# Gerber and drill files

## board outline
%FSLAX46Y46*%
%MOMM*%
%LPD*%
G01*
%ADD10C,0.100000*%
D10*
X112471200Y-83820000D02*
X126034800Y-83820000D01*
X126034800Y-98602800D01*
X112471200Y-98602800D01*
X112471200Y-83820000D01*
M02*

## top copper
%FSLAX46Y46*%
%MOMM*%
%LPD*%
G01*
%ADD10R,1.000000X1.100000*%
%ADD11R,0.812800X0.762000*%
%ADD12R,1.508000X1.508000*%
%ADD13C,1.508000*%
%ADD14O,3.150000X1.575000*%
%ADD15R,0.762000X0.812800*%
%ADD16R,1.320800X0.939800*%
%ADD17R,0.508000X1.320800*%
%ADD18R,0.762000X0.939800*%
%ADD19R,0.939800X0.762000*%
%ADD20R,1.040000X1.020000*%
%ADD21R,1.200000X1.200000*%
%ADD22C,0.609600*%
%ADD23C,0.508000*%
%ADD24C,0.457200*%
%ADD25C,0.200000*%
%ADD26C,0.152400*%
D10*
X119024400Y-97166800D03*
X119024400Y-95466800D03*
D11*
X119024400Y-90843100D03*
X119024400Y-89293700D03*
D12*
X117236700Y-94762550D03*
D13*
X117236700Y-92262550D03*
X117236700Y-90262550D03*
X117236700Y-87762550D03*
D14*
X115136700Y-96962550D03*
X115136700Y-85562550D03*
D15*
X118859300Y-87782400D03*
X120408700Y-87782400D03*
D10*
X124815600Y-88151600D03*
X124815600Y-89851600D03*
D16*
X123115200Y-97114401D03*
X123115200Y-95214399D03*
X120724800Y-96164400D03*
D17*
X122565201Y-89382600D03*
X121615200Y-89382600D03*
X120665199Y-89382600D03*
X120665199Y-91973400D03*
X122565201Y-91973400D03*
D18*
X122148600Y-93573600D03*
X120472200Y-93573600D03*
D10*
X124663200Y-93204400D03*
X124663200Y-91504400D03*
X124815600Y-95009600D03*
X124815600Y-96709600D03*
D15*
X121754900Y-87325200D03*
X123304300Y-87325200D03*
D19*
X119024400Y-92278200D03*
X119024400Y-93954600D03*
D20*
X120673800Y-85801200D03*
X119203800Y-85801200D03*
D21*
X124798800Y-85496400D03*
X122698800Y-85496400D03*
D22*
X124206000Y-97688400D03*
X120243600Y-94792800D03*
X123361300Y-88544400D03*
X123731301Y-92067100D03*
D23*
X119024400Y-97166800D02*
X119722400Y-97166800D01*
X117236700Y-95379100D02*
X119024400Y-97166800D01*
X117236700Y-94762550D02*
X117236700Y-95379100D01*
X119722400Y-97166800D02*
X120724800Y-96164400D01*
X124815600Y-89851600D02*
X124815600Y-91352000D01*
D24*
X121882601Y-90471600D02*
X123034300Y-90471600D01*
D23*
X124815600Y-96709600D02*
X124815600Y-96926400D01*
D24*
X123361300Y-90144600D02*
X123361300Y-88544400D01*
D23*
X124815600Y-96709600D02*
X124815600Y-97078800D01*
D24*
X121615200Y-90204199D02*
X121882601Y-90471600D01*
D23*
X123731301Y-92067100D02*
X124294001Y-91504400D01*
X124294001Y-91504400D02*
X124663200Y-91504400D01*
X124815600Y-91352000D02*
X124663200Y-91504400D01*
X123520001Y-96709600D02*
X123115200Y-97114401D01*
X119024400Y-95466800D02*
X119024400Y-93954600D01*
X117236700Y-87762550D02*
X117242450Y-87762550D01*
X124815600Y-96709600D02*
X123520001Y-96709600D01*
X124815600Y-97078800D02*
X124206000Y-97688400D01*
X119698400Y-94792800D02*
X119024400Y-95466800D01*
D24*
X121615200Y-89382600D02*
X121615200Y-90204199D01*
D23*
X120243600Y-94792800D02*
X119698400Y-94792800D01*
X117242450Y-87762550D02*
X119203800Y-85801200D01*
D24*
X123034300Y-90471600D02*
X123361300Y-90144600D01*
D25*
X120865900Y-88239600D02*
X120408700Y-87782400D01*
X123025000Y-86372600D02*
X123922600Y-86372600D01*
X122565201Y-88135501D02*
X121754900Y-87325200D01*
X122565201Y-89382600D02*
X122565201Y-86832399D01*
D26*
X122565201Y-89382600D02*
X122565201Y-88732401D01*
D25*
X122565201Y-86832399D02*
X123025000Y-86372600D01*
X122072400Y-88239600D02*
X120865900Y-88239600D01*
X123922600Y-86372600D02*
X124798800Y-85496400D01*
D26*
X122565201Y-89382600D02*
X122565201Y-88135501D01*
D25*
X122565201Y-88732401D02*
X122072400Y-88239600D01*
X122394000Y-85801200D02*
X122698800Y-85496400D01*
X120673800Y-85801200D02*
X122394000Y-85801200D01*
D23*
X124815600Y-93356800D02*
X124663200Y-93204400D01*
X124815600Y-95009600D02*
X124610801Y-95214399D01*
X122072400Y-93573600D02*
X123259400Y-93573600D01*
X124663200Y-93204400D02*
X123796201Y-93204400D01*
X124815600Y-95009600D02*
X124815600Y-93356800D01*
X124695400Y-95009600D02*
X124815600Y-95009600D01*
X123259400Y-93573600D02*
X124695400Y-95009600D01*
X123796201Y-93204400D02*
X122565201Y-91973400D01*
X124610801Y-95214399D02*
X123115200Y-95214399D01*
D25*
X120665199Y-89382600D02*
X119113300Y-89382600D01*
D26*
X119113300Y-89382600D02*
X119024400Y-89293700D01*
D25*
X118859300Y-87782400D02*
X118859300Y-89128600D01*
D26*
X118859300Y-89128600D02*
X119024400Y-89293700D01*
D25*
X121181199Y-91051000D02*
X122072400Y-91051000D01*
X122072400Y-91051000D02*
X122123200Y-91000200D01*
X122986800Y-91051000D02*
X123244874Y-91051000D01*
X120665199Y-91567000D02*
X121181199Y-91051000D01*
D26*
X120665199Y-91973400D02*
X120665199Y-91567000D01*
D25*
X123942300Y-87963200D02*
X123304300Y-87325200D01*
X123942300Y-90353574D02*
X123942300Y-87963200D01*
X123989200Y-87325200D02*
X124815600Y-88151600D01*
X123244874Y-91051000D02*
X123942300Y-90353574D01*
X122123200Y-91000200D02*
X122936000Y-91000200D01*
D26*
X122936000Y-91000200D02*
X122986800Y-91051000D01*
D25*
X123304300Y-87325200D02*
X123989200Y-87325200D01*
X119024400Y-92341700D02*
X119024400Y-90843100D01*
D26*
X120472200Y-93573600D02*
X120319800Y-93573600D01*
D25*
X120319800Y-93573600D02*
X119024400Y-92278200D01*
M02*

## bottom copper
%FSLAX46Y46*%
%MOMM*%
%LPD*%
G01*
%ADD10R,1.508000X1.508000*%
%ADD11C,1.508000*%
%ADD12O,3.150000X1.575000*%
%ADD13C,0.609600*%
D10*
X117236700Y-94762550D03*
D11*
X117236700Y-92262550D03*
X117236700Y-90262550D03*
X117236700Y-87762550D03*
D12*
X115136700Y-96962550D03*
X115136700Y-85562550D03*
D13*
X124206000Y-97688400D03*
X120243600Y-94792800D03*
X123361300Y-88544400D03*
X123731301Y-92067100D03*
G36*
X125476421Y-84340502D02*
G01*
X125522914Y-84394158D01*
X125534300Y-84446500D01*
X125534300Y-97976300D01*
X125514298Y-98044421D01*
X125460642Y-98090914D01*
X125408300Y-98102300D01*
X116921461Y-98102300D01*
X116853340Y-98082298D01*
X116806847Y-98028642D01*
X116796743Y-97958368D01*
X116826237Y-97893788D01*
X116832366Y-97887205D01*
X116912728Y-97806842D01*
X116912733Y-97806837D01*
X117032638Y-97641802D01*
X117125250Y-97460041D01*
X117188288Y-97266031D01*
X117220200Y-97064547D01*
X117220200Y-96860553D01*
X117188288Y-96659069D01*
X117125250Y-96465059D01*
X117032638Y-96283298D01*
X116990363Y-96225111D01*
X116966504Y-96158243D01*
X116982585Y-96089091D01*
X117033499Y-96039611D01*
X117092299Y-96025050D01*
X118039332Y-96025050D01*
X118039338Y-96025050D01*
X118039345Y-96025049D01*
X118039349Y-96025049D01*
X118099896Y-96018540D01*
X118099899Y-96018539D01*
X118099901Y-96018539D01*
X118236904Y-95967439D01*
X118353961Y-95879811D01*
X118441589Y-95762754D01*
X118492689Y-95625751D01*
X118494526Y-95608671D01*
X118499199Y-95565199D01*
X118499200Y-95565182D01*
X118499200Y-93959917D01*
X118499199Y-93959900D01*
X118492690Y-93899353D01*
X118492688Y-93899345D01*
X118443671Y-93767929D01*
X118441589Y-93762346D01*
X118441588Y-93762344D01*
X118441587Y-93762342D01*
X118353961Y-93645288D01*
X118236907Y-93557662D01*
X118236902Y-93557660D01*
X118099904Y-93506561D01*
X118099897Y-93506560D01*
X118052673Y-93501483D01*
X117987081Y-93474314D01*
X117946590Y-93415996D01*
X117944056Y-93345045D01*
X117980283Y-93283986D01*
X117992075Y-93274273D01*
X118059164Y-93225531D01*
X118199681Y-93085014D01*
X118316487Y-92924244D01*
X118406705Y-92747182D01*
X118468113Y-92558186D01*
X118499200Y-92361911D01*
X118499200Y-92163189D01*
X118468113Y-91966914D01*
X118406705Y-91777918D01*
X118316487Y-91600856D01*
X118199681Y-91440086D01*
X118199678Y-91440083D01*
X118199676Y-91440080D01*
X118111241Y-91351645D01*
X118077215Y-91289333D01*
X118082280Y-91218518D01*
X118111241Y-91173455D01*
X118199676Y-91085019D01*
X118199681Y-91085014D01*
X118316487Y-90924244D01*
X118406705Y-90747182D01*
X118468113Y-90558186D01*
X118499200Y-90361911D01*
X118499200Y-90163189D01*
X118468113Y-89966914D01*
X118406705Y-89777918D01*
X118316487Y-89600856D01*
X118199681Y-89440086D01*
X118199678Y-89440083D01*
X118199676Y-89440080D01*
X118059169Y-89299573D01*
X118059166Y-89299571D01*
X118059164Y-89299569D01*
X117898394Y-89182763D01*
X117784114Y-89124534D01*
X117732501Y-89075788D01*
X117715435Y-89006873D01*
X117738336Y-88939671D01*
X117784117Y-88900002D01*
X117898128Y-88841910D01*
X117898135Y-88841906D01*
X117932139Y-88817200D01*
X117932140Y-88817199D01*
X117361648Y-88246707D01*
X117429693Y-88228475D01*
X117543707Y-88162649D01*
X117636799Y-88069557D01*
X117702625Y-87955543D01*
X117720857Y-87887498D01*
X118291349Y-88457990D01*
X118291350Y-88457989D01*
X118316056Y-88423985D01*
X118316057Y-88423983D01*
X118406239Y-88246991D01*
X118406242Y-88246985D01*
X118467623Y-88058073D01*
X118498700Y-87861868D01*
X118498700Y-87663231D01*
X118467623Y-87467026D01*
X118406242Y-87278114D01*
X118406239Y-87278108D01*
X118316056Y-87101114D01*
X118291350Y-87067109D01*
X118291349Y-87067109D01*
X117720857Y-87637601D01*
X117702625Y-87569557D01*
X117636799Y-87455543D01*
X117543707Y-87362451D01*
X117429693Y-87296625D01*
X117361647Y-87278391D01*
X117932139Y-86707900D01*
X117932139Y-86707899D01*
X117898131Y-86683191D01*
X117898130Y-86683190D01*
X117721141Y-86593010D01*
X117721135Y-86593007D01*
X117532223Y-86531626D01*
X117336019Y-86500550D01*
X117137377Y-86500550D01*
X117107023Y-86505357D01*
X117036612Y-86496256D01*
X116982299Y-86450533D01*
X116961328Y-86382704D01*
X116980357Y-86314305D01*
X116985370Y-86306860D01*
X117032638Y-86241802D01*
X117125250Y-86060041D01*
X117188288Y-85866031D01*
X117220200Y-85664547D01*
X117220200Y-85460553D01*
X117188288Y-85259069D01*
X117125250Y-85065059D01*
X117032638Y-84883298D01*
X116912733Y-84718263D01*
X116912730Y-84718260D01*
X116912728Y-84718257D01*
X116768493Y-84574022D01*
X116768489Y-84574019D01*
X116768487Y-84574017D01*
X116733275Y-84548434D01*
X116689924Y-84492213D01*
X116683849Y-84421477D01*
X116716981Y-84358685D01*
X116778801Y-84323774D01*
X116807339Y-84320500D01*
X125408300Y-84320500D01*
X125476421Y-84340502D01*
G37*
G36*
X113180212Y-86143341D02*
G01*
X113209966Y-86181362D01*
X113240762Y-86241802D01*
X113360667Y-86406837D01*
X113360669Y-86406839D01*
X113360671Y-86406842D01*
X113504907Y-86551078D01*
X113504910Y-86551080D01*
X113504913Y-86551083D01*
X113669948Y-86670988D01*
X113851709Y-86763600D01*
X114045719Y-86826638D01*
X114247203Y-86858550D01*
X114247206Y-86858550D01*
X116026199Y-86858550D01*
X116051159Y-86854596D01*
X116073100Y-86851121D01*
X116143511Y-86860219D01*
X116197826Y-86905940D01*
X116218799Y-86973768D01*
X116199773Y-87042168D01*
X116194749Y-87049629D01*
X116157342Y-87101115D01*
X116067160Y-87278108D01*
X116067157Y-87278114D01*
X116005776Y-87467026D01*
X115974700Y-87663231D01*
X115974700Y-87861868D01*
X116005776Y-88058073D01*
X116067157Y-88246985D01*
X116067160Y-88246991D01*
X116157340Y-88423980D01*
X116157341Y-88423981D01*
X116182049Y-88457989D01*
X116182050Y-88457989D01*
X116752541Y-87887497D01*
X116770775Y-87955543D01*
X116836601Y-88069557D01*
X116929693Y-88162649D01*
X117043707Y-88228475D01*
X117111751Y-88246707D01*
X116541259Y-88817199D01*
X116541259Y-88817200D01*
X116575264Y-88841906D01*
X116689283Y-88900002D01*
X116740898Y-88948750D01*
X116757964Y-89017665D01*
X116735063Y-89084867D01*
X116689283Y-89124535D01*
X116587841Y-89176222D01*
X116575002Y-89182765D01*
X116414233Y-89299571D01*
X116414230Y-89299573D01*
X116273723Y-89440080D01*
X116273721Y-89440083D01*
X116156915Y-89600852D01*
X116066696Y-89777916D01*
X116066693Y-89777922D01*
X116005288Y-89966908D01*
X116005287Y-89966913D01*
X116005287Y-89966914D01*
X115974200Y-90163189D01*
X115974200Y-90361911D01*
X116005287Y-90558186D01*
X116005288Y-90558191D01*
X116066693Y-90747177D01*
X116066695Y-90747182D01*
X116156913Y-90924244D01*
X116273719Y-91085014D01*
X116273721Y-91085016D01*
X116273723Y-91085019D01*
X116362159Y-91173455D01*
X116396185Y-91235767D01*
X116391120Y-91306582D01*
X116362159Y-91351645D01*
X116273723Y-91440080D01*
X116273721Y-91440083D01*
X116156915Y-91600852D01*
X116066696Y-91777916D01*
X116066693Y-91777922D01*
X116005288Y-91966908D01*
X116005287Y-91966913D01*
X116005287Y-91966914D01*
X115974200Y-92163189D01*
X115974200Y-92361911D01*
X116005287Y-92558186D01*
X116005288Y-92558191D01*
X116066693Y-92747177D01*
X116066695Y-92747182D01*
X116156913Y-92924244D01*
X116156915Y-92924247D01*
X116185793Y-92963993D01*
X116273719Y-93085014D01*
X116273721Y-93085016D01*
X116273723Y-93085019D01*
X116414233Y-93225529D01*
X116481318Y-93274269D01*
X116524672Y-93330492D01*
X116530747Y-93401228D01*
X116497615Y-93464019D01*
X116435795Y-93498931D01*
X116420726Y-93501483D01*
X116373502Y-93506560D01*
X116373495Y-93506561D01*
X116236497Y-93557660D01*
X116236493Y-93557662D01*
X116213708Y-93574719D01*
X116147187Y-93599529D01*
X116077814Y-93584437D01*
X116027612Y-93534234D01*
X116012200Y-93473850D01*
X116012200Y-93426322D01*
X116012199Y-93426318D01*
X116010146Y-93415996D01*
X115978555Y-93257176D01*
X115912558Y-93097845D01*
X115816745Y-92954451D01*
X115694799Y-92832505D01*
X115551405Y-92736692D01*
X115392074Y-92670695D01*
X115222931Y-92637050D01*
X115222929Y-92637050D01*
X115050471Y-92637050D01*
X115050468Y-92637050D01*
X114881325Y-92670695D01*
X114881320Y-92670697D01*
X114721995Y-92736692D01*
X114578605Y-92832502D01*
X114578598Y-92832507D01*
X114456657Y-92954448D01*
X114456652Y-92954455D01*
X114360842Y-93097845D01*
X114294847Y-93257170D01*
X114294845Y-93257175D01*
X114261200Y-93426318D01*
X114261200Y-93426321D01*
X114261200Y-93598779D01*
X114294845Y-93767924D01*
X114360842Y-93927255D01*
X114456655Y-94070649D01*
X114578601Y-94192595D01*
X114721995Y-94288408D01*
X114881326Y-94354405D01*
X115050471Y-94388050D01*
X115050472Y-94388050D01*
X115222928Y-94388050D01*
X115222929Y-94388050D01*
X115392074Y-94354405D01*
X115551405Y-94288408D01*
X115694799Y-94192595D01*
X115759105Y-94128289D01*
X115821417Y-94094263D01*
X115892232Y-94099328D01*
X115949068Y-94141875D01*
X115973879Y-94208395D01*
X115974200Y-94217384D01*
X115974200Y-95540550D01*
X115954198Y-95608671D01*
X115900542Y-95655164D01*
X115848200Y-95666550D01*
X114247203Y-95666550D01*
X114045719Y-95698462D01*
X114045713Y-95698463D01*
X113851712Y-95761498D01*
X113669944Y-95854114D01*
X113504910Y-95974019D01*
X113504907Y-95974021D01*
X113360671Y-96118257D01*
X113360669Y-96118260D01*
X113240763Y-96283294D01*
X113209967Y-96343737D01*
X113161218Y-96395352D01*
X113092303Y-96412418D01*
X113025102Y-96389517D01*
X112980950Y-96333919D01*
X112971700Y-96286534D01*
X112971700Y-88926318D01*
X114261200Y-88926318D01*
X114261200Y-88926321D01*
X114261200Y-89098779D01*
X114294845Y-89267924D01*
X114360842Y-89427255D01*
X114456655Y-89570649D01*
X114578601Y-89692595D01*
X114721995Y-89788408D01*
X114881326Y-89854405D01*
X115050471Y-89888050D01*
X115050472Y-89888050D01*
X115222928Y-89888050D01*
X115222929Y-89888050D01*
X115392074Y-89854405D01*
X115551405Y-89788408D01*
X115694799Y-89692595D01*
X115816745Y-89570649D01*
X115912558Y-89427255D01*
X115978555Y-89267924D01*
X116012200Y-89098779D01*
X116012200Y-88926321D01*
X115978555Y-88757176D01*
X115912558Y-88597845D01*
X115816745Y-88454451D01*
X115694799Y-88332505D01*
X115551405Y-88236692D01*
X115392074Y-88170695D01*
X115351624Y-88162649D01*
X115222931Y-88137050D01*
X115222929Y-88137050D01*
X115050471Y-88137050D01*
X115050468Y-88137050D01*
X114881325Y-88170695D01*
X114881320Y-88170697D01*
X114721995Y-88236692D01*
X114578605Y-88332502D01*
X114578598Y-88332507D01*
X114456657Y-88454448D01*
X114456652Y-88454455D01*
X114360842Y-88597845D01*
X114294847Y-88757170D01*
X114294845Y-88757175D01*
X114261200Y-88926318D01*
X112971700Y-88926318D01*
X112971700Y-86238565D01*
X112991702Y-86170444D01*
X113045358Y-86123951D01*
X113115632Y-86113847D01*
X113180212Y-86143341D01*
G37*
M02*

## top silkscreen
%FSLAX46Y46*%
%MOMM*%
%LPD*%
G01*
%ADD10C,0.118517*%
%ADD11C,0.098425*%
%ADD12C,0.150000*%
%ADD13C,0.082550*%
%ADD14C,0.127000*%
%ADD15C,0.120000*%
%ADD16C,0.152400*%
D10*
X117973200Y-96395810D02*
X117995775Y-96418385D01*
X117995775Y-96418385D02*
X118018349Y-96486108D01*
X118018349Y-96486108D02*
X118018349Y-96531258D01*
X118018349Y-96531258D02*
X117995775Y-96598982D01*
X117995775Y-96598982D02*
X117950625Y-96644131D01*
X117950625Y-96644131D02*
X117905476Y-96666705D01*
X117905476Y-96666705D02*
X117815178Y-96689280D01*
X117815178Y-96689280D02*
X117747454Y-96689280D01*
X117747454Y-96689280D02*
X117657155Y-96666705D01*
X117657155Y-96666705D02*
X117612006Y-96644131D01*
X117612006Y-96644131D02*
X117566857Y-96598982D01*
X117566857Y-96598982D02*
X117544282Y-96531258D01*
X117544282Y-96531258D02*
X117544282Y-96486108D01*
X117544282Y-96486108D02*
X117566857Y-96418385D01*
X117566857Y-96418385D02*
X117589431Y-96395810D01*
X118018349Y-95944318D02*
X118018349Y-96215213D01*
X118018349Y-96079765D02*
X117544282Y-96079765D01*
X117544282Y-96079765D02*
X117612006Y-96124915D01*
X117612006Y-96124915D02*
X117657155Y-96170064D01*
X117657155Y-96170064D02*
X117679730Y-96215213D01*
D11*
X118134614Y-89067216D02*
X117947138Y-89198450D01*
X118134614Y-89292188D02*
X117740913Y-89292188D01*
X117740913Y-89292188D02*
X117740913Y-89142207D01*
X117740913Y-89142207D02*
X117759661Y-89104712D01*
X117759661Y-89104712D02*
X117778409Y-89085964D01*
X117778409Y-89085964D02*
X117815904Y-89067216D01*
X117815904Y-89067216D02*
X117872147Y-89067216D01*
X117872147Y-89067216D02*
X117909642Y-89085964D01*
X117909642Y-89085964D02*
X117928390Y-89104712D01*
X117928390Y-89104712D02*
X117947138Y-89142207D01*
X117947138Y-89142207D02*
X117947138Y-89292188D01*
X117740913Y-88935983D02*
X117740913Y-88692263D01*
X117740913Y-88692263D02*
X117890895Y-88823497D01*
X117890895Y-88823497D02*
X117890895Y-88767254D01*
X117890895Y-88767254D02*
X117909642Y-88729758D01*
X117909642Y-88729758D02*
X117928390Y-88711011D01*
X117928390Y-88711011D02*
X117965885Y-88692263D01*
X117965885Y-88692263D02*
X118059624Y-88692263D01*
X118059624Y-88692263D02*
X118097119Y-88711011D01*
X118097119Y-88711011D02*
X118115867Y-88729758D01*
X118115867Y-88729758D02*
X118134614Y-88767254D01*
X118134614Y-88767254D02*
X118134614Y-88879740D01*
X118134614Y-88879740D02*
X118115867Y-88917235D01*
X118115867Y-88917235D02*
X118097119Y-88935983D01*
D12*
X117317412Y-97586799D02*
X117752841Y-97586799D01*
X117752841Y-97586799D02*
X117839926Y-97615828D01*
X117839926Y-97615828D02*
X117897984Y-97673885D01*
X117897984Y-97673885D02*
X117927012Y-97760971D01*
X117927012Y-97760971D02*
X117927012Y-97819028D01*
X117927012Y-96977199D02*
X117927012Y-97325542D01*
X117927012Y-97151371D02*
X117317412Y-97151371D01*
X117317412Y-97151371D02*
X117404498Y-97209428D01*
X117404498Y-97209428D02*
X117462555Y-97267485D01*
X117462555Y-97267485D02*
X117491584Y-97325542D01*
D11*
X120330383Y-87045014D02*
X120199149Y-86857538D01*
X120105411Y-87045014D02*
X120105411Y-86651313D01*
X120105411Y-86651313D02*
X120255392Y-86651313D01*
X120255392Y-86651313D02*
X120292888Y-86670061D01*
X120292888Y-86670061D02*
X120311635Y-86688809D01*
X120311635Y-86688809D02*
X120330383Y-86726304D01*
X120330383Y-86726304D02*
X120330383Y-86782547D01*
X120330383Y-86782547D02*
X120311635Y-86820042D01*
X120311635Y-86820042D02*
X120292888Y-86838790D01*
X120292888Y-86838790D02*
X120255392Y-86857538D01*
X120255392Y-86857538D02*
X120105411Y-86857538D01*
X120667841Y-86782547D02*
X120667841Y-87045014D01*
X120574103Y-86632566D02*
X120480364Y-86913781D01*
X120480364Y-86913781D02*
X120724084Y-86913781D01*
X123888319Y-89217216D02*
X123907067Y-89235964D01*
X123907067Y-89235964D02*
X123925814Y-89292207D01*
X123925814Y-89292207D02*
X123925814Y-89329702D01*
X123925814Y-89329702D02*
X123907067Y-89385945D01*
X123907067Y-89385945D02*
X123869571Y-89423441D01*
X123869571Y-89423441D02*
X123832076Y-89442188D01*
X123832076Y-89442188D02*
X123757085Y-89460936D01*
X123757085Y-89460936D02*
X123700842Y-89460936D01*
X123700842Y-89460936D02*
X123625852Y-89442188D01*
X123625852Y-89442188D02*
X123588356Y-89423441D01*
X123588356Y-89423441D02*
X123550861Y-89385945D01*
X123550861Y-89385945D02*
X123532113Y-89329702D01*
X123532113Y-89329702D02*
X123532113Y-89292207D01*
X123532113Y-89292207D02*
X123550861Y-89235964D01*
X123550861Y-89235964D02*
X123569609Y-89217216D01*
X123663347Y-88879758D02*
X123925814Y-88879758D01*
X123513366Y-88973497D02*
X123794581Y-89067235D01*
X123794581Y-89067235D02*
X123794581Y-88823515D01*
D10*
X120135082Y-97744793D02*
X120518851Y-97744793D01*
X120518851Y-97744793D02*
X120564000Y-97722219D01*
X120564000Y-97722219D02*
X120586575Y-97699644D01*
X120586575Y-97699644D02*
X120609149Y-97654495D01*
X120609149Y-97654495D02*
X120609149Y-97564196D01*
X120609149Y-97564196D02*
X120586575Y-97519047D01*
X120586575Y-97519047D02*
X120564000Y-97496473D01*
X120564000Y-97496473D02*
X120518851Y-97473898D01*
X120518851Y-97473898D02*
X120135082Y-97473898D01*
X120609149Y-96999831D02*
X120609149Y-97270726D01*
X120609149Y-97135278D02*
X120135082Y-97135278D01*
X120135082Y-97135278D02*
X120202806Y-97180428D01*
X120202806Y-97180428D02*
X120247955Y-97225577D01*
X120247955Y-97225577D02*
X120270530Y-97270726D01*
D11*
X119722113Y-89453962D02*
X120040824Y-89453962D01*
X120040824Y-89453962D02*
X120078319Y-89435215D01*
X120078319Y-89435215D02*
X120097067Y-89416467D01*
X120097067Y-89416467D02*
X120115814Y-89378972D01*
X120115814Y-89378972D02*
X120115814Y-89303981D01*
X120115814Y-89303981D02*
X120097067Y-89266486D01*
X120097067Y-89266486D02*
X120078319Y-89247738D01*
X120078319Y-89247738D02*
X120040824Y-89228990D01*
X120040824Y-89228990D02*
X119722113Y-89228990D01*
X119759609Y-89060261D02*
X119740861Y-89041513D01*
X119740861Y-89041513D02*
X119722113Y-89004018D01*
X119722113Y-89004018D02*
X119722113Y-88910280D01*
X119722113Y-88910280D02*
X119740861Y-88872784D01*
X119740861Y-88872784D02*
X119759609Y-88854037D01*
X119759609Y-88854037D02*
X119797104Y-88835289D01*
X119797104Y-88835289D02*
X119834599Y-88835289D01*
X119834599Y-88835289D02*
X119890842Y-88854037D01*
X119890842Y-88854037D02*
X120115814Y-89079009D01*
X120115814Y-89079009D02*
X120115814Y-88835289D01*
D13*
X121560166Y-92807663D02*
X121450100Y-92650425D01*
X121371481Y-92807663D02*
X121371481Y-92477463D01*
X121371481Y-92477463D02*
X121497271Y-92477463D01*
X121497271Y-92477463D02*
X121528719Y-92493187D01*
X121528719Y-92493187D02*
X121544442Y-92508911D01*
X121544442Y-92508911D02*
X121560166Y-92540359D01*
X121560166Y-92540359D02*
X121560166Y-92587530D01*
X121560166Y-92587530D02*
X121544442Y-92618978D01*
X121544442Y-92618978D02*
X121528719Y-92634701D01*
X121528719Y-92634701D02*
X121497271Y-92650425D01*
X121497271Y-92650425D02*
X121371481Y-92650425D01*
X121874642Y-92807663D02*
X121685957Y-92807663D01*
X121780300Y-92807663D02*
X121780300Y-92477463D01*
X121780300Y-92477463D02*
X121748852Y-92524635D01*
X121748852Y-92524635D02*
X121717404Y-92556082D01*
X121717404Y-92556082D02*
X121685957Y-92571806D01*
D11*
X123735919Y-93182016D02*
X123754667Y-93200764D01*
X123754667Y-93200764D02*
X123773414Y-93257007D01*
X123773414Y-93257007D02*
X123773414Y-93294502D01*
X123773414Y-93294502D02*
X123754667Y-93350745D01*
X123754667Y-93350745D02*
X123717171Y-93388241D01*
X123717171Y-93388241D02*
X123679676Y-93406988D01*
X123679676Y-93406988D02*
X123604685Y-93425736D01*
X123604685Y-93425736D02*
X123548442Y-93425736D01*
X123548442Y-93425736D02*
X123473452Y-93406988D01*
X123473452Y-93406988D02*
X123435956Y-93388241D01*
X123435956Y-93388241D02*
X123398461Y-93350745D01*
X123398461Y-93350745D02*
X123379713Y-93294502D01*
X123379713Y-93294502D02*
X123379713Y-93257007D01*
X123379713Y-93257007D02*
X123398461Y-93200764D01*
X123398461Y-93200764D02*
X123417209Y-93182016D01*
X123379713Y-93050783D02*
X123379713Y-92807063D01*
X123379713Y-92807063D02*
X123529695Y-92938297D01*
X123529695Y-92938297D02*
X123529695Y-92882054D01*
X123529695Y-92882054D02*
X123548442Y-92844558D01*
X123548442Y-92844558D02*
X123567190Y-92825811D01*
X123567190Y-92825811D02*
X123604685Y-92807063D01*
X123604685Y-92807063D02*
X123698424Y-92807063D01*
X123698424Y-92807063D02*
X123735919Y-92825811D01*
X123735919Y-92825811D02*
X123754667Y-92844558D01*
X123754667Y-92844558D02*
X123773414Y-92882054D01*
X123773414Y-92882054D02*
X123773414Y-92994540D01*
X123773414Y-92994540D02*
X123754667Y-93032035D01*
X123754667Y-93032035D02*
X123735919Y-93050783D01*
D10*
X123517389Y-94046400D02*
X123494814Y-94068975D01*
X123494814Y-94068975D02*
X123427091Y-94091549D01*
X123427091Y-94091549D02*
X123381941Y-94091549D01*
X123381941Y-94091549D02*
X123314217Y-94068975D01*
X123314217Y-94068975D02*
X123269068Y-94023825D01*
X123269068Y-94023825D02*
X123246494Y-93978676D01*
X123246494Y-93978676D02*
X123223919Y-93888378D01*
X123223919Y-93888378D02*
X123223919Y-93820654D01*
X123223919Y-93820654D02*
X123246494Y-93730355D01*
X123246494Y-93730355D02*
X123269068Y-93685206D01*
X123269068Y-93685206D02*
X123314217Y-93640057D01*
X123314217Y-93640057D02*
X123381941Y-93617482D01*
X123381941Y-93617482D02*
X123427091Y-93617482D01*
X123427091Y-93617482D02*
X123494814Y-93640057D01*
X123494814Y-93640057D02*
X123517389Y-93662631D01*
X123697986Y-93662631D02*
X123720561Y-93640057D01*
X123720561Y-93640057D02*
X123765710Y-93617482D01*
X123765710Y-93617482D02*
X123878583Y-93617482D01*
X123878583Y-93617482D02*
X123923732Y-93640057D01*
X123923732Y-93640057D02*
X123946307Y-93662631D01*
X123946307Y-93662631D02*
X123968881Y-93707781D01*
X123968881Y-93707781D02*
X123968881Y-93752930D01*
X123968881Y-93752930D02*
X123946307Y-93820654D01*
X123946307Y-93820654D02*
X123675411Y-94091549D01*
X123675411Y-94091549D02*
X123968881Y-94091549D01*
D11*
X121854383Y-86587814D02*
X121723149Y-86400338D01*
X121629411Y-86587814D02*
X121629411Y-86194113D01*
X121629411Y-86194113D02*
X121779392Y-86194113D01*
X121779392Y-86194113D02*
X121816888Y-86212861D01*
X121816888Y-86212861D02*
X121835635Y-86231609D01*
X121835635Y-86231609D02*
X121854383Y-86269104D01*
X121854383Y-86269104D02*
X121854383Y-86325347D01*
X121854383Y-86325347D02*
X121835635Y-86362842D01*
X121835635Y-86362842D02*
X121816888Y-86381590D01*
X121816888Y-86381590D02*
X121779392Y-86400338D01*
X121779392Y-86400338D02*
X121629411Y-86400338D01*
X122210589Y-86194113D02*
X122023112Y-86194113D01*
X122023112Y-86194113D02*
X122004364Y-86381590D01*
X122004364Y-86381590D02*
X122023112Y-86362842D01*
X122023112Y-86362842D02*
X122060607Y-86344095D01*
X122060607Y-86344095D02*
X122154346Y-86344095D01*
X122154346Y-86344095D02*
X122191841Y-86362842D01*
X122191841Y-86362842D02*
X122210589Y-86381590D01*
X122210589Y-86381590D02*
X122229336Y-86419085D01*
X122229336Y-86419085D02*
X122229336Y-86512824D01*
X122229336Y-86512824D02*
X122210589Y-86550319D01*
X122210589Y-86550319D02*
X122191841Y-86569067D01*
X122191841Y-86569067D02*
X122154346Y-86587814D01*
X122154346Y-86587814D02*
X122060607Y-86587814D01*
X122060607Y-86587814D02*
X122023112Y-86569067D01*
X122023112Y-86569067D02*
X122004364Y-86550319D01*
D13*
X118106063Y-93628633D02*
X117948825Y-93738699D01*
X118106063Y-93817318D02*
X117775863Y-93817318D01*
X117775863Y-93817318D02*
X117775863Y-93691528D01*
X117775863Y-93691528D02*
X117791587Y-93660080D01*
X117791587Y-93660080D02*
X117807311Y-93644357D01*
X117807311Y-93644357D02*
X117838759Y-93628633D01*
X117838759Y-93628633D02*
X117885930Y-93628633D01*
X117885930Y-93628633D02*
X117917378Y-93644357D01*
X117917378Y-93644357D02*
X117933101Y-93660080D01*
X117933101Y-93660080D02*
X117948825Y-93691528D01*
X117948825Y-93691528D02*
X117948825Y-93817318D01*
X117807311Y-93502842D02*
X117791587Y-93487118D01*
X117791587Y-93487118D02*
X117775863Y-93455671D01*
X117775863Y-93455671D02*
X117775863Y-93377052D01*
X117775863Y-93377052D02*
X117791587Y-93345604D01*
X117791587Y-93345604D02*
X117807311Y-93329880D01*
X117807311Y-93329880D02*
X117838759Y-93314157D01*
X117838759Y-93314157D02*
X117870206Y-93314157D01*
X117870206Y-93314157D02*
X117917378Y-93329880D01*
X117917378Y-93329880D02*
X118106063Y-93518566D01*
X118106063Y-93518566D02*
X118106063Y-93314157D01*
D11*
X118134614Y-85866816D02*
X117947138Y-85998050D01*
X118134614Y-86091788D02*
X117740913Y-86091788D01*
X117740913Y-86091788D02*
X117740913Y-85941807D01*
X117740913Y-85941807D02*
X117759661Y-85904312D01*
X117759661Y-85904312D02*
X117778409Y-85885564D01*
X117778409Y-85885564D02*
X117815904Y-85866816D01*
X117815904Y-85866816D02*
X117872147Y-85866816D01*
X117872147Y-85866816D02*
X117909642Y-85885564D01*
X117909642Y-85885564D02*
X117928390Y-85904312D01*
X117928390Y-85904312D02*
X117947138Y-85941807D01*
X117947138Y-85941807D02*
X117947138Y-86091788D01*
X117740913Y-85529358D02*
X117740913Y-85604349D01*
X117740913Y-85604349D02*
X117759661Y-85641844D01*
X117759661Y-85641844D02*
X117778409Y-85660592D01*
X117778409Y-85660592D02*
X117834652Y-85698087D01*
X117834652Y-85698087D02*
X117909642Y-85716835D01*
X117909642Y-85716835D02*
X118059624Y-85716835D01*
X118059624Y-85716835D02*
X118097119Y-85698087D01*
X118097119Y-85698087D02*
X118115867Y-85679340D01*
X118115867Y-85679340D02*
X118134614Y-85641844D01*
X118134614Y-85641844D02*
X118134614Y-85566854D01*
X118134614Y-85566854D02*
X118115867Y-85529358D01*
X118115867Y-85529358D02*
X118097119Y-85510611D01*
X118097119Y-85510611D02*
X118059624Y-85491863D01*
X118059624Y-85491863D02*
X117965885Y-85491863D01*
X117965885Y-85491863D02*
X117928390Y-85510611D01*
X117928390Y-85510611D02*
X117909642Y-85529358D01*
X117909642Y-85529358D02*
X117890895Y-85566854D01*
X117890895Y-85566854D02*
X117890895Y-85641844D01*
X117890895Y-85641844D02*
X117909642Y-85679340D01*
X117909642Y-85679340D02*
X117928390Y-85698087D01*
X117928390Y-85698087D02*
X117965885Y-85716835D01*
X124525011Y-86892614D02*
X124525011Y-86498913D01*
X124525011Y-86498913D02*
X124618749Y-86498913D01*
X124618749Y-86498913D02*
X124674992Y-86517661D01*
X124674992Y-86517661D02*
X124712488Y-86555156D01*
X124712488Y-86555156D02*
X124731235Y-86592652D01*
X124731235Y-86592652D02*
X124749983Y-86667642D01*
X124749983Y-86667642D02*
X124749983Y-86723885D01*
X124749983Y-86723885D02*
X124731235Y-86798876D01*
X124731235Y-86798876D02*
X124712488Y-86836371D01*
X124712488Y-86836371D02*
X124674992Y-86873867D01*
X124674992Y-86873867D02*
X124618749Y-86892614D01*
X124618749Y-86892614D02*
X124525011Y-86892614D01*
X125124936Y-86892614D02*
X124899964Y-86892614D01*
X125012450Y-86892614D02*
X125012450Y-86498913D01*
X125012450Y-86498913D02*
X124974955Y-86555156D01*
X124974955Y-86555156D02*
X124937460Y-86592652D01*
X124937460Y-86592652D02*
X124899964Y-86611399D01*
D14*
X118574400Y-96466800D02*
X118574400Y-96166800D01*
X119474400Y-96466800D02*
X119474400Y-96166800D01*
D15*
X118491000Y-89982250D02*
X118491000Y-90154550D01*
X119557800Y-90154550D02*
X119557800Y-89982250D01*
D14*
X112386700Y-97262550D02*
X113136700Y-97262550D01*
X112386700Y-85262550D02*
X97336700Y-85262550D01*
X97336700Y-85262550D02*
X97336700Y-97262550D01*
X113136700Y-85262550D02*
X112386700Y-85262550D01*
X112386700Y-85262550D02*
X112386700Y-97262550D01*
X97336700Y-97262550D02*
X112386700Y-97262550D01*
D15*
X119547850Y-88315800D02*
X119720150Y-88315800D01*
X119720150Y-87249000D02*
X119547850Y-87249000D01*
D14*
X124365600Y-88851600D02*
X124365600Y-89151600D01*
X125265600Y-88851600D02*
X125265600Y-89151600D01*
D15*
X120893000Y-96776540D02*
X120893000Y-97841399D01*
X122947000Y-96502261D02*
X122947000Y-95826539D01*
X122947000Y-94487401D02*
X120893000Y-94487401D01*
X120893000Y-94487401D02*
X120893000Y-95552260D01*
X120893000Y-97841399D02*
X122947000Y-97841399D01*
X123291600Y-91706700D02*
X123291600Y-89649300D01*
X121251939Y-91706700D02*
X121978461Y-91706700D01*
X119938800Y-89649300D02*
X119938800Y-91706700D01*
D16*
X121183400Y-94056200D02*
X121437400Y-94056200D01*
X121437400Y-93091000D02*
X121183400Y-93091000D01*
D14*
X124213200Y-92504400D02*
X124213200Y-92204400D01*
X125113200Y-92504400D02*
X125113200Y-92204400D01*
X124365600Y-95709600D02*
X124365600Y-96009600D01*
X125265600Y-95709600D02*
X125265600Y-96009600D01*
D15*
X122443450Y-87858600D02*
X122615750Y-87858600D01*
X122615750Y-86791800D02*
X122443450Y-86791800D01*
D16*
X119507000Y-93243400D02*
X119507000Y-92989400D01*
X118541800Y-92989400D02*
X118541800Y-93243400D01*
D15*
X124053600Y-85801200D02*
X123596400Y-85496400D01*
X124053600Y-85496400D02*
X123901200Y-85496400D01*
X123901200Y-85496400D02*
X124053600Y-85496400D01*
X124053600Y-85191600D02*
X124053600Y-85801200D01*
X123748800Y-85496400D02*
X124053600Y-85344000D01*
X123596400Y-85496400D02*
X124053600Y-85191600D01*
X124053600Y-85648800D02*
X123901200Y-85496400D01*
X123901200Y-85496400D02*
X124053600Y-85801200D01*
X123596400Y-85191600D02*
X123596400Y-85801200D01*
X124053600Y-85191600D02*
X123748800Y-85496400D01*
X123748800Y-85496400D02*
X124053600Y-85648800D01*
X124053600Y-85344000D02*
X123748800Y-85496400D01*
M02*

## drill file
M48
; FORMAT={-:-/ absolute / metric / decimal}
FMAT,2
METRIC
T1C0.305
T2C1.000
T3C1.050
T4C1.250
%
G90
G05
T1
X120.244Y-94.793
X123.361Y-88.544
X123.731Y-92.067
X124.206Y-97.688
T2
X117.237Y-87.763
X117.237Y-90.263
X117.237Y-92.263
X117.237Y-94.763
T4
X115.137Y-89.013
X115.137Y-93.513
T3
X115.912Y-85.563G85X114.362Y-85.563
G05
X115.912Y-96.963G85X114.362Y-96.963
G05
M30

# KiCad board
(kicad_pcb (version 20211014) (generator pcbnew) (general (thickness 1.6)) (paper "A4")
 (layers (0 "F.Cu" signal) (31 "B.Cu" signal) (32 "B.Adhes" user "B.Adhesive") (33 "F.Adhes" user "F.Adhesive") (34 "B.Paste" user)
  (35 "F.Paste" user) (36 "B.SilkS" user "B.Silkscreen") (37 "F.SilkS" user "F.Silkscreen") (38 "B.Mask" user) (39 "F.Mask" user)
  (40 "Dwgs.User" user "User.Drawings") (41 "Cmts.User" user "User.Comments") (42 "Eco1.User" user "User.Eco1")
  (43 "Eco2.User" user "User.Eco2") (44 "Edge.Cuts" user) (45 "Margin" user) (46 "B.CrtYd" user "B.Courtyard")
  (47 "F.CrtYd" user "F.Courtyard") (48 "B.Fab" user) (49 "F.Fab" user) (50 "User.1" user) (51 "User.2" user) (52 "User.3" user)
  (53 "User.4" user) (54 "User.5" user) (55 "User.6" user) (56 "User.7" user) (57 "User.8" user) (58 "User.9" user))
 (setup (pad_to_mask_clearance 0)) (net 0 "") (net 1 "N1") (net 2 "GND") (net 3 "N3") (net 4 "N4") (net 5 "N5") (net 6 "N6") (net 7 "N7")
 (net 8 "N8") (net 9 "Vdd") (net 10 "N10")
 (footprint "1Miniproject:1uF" (layer "F.Cu") (at 119.0244 96.3168 90)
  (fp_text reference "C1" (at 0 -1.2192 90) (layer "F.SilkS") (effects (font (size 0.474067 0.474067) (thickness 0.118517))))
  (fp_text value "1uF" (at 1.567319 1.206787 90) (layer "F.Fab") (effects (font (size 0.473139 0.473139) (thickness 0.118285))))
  (fp_line (start -0.15 -0.45) (end 0.15 -0.45) (layer "F.SilkS") (width 0.127))
  (fp_line (start -0.15 0.45) (end 0.15 0.45) (layer "F.SilkS") (width 0.127))
  (pad "1" smd rect (at -0.85 0 90) (size 1.1 1) (layers "F.Cu" "F.Paste" "F.Mask") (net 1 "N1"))
  (pad "2" smd rect (at 0.85 0 90) (size 1.1 1) (layers "F.Cu" "F.Paste" "F.Mask") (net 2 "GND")))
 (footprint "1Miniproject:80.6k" (layer "F.Cu") (at 119.0244 90.0684 90)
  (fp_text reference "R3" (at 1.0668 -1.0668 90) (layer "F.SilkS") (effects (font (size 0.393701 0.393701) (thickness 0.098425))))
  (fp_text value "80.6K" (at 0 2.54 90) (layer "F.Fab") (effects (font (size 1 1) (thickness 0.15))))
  (fp_line (start 0.08615 -0.5334) (end -0.08615 -0.5334) (layer "F.SilkS") (width 0.12))
  (fp_line (start -0.08615 0.5334) (end 0.08615 0.5334) (layer "F.SilkS") (width 0.12))
  (pad "1" smd rect (at -0.7747 0 90) (size 0.762 0.8128) (layers "F.Cu" "F.Paste" "F.Mask") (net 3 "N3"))
  (pad "2" smd rect (at 0.7747 0 90) (size 0.762 0.8128) (layers "F.Cu" "F.Paste" "F.Mask") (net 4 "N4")))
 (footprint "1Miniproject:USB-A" (layer "F.Cu") (at 115.1367 91.26255 -90)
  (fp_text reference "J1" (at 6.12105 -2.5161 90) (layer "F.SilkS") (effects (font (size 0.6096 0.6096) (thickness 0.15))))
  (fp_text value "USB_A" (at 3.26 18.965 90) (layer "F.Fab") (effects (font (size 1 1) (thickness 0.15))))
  (fp_line (start 6 2.75) (end 6 2) (layer "F.SilkS") (width 0.127))
  (fp_line (start -6 2.75) (end -6 17.8) (layer "F.SilkS") (width 0.127))
  (fp_line (start -6 17.8) (end 6 17.8) (layer "F.SilkS") (width 0.127))
  (fp_line (start -6 2) (end -6 2.75) (layer "F.SilkS") (width 0.127))
  (fp_line (start -6 2.75) (end 6 2.75) (layer "F.SilkS") (width 0.127))
  (fp_line (start 6 17.8) (end 6 2.75) (layer "F.SilkS") (width 0.127))
  (pad "" np_thru_hole circle (at -2.25 0 270) (size 1.25 1.25) (drill 1.25) (layers *.Cu *.Mask))
  (pad "" np_thru_hole circle (at 2.25 0 270) (size 1.25 1.25) (drill 1.25) (layers *.Cu *.Mask))
  (pad "1" thru_hole rect (at 3.5 -2.1 270) (size 1.508 1.508) (drill 1) (layers *.Cu *.Mask) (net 1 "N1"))
  (pad "2" thru_hole circle (at 1 -2.1 270) (size 1.508 1.508) (drill 1) (layers *.Cu *.Mask) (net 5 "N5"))
  (pad "3" thru_hole circle (at -1 -2.1 270) (size 1.508 1.508) (drill 1) (layers *.Cu *.Mask) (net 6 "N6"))
  (pad "4" thru_hole circle (at -3.5 -2.1 270) (size 1.508 1.508) (drill 1) (layers *.Cu *.Mask) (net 2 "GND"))
  (pad "S1" thru_hole oval (at 5.7 0 270) (size 1.575 3.15) (drill oval 1.05 2.6) (layers *.Cu *.Mask))
  (pad "S2" thru_hole oval (at -5.7 0 270) (size 1.575 3.15) (drill oval 1.05 2.6) (layers *.Cu *.Mask)))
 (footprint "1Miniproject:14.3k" (layer "F.Cu") (at 119.634 87.7824)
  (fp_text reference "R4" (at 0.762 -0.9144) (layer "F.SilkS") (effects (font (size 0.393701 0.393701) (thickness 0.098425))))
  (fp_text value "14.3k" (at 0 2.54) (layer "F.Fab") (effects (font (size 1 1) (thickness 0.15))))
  (fp_line (start -0.08615 0.5334) (end 0.08615 0.5334) (layer "F.SilkS") (width 0.12))
  (fp_line (start 0.08615 -0.5334) (end -0.08615 -0.5334) (layer "F.SilkS") (width 0.12))
  (pad "1" smd rect (at -0.7747 0) (size 0.762 0.8128) (layers "F.Cu" "F.Paste" "F.Mask") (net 4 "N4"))
  (pad "2" smd rect (at 0.7747 0) (size 0.762 0.8128) (layers "F.Cu" "F.Paste" "F.Mask") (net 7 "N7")))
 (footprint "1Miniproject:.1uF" (layer "F.Cu") (at 124.8156 89.0016 -90)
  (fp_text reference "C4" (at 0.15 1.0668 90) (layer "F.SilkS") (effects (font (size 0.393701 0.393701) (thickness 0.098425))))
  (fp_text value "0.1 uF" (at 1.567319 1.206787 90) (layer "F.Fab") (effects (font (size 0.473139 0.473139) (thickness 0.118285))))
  (fp_line (start -0.15 0.45) (end 0.15 0.45) (layer "F.SilkS") (width 0.127))
  (fp_line (start -0.15 -0.45) (end 0.15 -0.45) (layer "F.SilkS") (width 0.127))
  (pad "1" smd rect (at -0.85 0 270) (size 1.1 1) (layers "F.Cu" "F.Paste" "F.Mask") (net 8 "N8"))
  (pad "2" smd rect (at 0.85 0 270) (size 1.1 1) (layers "F.Cu" "F.Paste" "F.Mask") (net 2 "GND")))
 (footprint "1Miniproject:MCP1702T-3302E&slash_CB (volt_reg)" (layer "F.Cu") (at 121.92 96.1644 90)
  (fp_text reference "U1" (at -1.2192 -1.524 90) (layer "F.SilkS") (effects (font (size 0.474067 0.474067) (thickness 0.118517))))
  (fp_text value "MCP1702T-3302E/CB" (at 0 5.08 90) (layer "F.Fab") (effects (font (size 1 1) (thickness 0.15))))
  (fp_line (start -0.61214 -1.027) (end -1.676999 -1.027) (layer "F.SilkS") (width 0.12))
  (fp_line (start -0.337861 1.027) (end 0.337861 1.027) (layer "F.SilkS") (width 0.12))
  (fp_line (start 1.676999 1.027) (end 1.676999 -1.027) (layer "F.SilkS") (width 0.12))
  (fp_line (start 1.676999 -1.027) (end 0.61214 -1.027) (layer "F.SilkS") (width 0.12))
  (fp_line (start -1.676999 -1.027) (end -1.676999 1.027) (layer "F.SilkS") (width 0.12))
  (pad "1" smd rect (at -0.950001 1.1952 90) (size 0.9398 1.3208) (layers "F.Cu" "F.Paste" "F.Mask") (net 2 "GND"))
  (pad "2" smd rect (at 0.950001 1.1952 90) (size 0.9398 1.3208) (layers "F.Cu" "F.Paste" "F.Mask") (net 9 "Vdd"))
  (pad "3" smd rect (at 0 -1.1952 90) (size 0.9398 1.3208) (layers "F.Cu" "F.Paste" "F.Mask") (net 1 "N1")))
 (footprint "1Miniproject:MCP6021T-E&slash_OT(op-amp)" (layer "F.Cu") (at 121.6152 90.678 -90)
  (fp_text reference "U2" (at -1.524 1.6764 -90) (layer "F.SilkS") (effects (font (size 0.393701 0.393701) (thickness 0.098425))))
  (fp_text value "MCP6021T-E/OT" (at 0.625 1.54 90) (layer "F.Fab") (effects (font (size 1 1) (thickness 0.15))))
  (fp_line (start 1.0287 -1.6764) (end -1.0287 -1.6764) (layer "F.SilkS") (width 0.12))
  (fp_line (start 1.0287 0.363261) (end 1.0287 -0.363261) (layer "F.SilkS") (width 0.12))
  (fp_line (start -1.0287 1.6764) (end 1.0287 1.6764) (layer "F.SilkS") (width 0.12))
  (pad "1" smd rect (at -1.2954 -0.950001 270) (size 1.3208 0.508) (layers "F.Cu" "F.Paste" "F.Mask") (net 7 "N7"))
  (pad "2" smd rect (at -1.2954 0 270) (size 1.3208 0.508) (layers "F.Cu" "F.Paste" "F.Mask") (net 2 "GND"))
  (pad "3" smd rect (at -1.2954 0.950001 270) (size 1.3208 0.508) (layers "F.Cu" "F.Paste" "F.Mask") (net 4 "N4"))
  (pad "4" smd rect (at 1.2954 0.950001 270) (size 1.3208 0.508) (layers "F.Cu" "F.Paste" "F.Mask") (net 8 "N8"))
  (pad "5" smd rect (at 1.2954 -0.950001 270) (size 1.3208 0.508) (layers "F.Cu" "F.Paste" "F.Mask") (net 9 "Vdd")))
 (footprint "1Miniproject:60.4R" (layer "F.Cu") (at 121.3104 93.5736 180)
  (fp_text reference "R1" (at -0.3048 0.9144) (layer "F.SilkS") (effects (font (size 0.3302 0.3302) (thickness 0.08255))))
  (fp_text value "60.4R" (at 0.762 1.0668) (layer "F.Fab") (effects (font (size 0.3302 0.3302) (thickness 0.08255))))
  (fp_line (start 0.127 -0.4826) (end -0.127 -0.4826) (layer "F.SilkS") (width 0.1524))
  (fp_line (start -0.127 0.4826) (end 0.127 0.4826) (layer "F.SilkS") (width 0.1524))
  (pad "1" smd rect (at -0.8382 0 180) (size 0.762 0.9398) (layers "F.Cu" "F.Paste" "F.Mask") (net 9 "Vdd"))
  (pad "2" smd rect (at 0.8382 0 180) (size 0.762 0.9398) (layers "F.Cu" "F.Paste" "F.Mask") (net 3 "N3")))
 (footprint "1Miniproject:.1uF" (layer "F.Cu") (at 124.6632 92.3544 90)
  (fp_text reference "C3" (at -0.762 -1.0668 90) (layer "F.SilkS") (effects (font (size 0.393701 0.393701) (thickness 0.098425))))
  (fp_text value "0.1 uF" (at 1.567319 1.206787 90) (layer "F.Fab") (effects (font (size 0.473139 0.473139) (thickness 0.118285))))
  (fp_line (start -0.15 -0.45) (end 0.15 -0.45) (layer "F.SilkS") (width 0.127))
  (fp_line (start -0.15 0.45) (end 0.15 0.45) (layer "F.SilkS") (width 0.127))
  (pad "1" smd rect (at -0.85 0 90) (size 1.1 1) (layers "F.Cu" "F.Paste" "F.Mask") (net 9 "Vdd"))
  (pad "2" smd rect (at 0.85 0 90) (size 1.1 1) (layers "F.Cu" "F.Paste" "F.Mask") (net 2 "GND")))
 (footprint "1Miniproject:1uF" (layer "F.Cu") (at 124.8156 95.8596 -90)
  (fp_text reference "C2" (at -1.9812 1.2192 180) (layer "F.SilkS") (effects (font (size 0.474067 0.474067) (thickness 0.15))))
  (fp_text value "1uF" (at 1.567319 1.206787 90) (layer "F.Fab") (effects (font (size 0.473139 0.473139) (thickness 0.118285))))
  (fp_line (start -0.15 0.45) (end 0.15 0.45) (layer "F.SilkS") (width 0.127))
  (fp_line (start -0.15 -0.45) (end 0.15 -0.45) (layer "F.SilkS") (width 0.127))
  (pad "1" smd rect (at -0.85 0 270) (size 1.1 1) (layers "F.Cu" "F.Paste" "F.Mask") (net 9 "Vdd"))
  (pad "2" smd rect (at 0.85 0 270) (size 1.1 1) (layers "F.Cu" "F.Paste" "F.Mask") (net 2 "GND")))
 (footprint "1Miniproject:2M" (layer "F.Cu") (at 122.5296 87.3252)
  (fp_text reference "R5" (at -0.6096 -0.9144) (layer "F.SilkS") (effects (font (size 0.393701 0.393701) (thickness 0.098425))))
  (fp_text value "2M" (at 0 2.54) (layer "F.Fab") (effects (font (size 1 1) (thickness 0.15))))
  (fp_line (start -0.08615 0.5334) (end 0.08615 0.5334) (layer "F.SilkS") (width 0.12))
  (fp_line (start 0.08615 -0.5334) (end -0.08615 -0.5334) (layer "F.SilkS") (width 0.12))
  (pad "1" smd rect (at -0.7747 0) (size 0.762 0.8128) (layers "F.Cu" "F.Paste" "F.Mask") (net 7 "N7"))
  (pad "2" smd rect (at 0.7747 0) (size 0.762 0.8128) (layers "F.Cu" "F.Paste" "F.Mask") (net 8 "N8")))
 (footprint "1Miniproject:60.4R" (layer "F.Cu") (at 119.0244 93.1164 -90)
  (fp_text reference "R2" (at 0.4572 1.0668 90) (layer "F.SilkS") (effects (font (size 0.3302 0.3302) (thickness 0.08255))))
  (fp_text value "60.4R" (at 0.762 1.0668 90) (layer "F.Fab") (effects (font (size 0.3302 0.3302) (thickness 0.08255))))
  (fp_line (start 0.127 -0.4826) (end -0.127 -0.4826) (layer "F.SilkS") (width 0.1524))
  (fp_line (start -0.127 0.4826) (end 0.127 0.4826) (layer "F.SilkS") (width 0.1524))
  (pad "1" smd rect (at -0.8382 0 270) (size 0.762 0.9398) (layers "F.Cu" "F.Paste" "F.Mask") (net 3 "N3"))
  (pad "2" smd rect (at 0.8382 0 270) (size 0.762 0.9398) (layers "F.Cu" "F.Paste" "F.Mask") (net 2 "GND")))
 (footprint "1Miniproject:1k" (layer "F.Cu") (at 119.9388 85.8012 180)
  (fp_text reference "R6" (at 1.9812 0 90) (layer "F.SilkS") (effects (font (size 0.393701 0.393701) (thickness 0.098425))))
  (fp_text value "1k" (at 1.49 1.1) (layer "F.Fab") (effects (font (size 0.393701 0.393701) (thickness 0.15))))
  (pad "1" smd rect (at -0.735 0 180) (size 1.04 1.02) (layers "F.Cu" "F.Paste" "F.Mask") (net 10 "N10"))
  (pad "2" smd rect (at 0.735 0 180) (size 1.04 1.02) (layers "F.Cu" "F.Paste" "F.Mask") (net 2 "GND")))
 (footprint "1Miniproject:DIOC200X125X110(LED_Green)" (layer "F.Cu") (at 123.7488 85.4964)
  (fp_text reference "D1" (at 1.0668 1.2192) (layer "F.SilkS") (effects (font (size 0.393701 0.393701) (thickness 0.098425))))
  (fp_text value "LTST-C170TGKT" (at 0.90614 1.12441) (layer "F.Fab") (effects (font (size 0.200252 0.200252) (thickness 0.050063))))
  (fp_line (start 0.3048 0.3048) (end -0.1524 0) (layer "F.SilkS") (width 0.12))
  (fp_line (start 0.3048 0) (end 0.1524 0) (layer "F.SilkS") (width 0.12))
  (fp_line (start 0.1524 0) (end 0.3048 0) (layer "F.SilkS") (width 0.12))
  (fp_line (start 0.3048 -0.3048) (end 0.3048 0.3048) (layer "F.SilkS") (width 0.12))
  (fp_line (start 0 0) (end 0.3048 -0.1524) (layer "F.SilkS") (width 0.12))
  (fp_line (start -0.1524 0) (end 0.3048 -0.3048) (layer "F.SilkS") (width 0.12))
  (fp_line (start 0.3048 0.1524) (end 0.1524 0) (layer "F.SilkS") (width 0.12))
  (fp_line (start 0.1524 0) (end 0.3048 0.3048) (layer "F.SilkS") (width 0.12))
  (fp_line (start -0.1524 -0.3048) (end -0.1524 0.3048) (layer "F.SilkS") (width 0.12))
  (fp_line (start 0.3048 -0.3048) (end 0 0) (layer "F.SilkS") (width 0.12))
  (fp_line (start 0 0) (end 0.3048 0.1524) (layer "F.SilkS") (width 0.12))
  (fp_line (start 0.3048 -0.1524) (end 0 0) (layer "F.SilkS") (width 0.12))
  (pad "+" smd rect (at 1.05 0) (size 1.2 1.2) (layers "F.Cu" "F.Paste" "F.Mask") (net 7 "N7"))
  (pad "-" smd rect (at -1.05 0) (size 1.2 1.2) (layers "F.Cu" "F.Paste" "F.Mask") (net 10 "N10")))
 (gr_rect (start 112.4712 83.82) (end 126.0348 98.6028) (layer "Edge.Cuts") (width 0.1) (fill none))
 (segment (start 119.0244 97.1668) (end 119.7224 97.1668) (width 0.508) (layer "F.Cu") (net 1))
 (segment (start 117.2367 95.3791) (end 119.0244 97.1668) (width 0.508) (layer "F.Cu") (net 1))
 (segment (start 117.2367 94.76255) (end 117.2367 95.3791) (width 0.508) (layer "F.Cu") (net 1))
 (segment (start 119.7224 97.1668) (end 120.7248 96.1644) (width 0.508) (layer "F.Cu") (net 1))
 (segment (start 124.8156 89.8516) (end 124.8156 91.352) (width 0.508) (layer "F.Cu") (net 2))
 (segment (start 121.882601 90.4716) (end 123.0343 90.4716) (width 0.4572) (layer "F.Cu") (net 2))
 (segment (start 124.8156 96.7096) (end 124.8156 96.9264) (width 0.508) (layer "F.Cu") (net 2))
 (segment (start 123.3613 90.1446) (end 123.3613 88.5444) (width 0.4572) (layer "F.Cu") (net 2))
 (segment (start 124.8156 96.7096) (end 124.8156 97.0788) (width 0.508) (layer "F.Cu") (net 2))
 (segment (start 121.6152 90.204199) (end 121.882601 90.4716) (width 0.4572) (layer "F.Cu") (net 2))
 (segment (start 123.731301 92.0671) (end 124.294001 91.5044) (width 0.508) (layer "F.Cu") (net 2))
 (segment (start 124.294001 91.5044) (end 124.6632 91.5044) (width 0.508) (layer "F.Cu") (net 2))
 (segment (start 124.8156 91.352) (end 124.6632 91.5044) (width 0.508) (layer "F.Cu") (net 2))
 (segment (start 123.520001 96.7096) (end 123.1152 97.114401) (width 0.508) (layer "F.Cu") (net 2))
 (segment (start 119.0244 95.4668) (end 119.0244 93.9546) (width 0.508) (layer "F.Cu") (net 2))
 (segment (start 117.2367 87.76255) (end 117.24245 87.76255) (width 0.508) (layer "F.Cu") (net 2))
 (segment (start 124.8156 96.7096) (end 123.520001 96.7096) (width 0.508) (layer "F.Cu") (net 2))
 (segment (start 124.8156 97.0788) (end 124.206 97.6884) (width 0.508) (layer "F.Cu") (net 2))
 (segment (start 119.6984 94.7928) (end 119.0244 95.4668) (width 0.508) (layer "F.Cu") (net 2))
 (segment (start 121.6152 89.3826) (end 121.6152 90.204199) (width 0.4572) (layer "F.Cu") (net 2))
 (segment (start 120.2436 94.7928) (end 119.6984 94.7928) (width 0.508) (layer "F.Cu") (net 2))
 (segment (start 117.24245 87.76255) (end 119.2038 85.8012) (width 0.508) (layer "F.Cu") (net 2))
 (segment (start 123.0343 90.4716) (end 123.3613 90.1446) (width 0.4572) (layer "F.Cu") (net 2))
 (via (at 124.206 97.6884) (size 0.6096) (drill 0.3048) (layers "F.Cu" "B.Cu") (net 2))
 (via (at 120.2436 94.7928) (size 0.6096) (drill 0.3048) (layers "F.Cu" "B.Cu") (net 2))
 (via (at 123.3613 88.5444) (size 0.6096) (drill 0.3048) (layers "F.Cu" "B.Cu") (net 2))
 (via (at 123.731301 92.0671) (size 0.6096) (drill 0.3048) (layers "F.Cu" "B.Cu") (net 2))
 (segment (start 120.8659 88.2396) (end 120.4087 87.7824) (width 0.2) (layer "F.Cu") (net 7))
 (segment (start 123.025 86.3726) (end 123.9226 86.3726) (width 0.2) (layer "F.Cu") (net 7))
 (segment (start 122.565201 88.135501) (end 121.7549 87.3252) (width 0.2) (layer "F.Cu") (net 7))
 (segment (start 122.565201 89.3826) (end 122.565201 86.832399) (width 0.2) (layer "F.Cu") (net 7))
 (segment (start 122.565201 89.3826) (end 122.565201 88.732401) (width 0.1524) (layer "F.Cu") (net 7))
 (segment (start 122.565201 86.832399) (end 123.025 86.3726) (width 0.2) (layer "F.Cu") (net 7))
 (segment (start 122.0724 88.2396) (end 120.8659 88.2396) (width 0.2) (layer "F.Cu") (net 7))
 (segment (start 123.9226 86.3726) (end 124.7988 85.4964) (width 0.2) (layer "F.Cu") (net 7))
 (segment (start 122.565201 89.3826) (end 122.565201 88.135501) (width 0.1524) (layer "F.Cu") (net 7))
 (segment (start 122.565201 88.732401) (end 122.0724 88.2396) (width 0.2) (layer "F.Cu") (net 7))
 (segment (start 122.394 85.8012) (end 122.6988 85.4964) (width 0.2) (layer "F.Cu") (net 10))
 (segment (start 120.6738 85.8012) (end 122.394 85.8012) (width 0.2) (layer "F.Cu") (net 10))
 (segment (start 124.8156 93.3568) (end 124.6632 93.2044) (width 0.508) (layer "F.Cu") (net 9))
 (segment (start 124.8156 95.0096) (end 124.610801 95.214399) (width 0.508) (layer "F.Cu") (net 9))
 (segment (start 122.0724 93.5736) (end 123.2594 93.5736) (width 0.508) (layer "F.Cu") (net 9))
 (segment (start 124.6632 93.2044) (end 123.796201 93.2044) (width 0.508) (layer "F.Cu") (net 9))
 (segment (start 124.8156 95.0096) (end 124.8156 93.3568) (width 0.508) (layer "F.Cu") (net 9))
 (segment (start 124.6954 95.0096) (end 124.8156 95.0096) (width 0.508) (layer "F.Cu") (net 9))
 (segment (start 123.2594 93.5736) (end 124.6954 95.0096) (width 0.508) (layer "F.Cu") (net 9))
 (segment (start 123.796201 93.2044) (end 122.565201 91.9734) (width 0.508) (layer "F.Cu") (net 9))
 (segment (start 124.610801 95.214399) (end 123.1152 95.214399) (width 0.508) (layer "F.Cu") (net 9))
 (segment (start 120.665199 89.3826) (end 119.1133 89.3826) (width 0.2) (layer "F.Cu") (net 4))
 (segment (start 119.1133 89.3826) (end 119.0244 89.2937) (width 0.1524) (layer "F.Cu") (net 4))
 (segment (start 118.8593 87.7824) (end 118.8593 89.1286) (width 0.2) (layer "F.Cu") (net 4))
 (segment (start 118.8593 89.1286) (end 119.0244 89.2937) (width 0.1524) (layer "F.Cu") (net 4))
 (segment (start 121.181199 91.051) (end 122.0724 91.051) (width 0.2) (layer "F.Cu") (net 8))
 (segment (start 122.0724 91.051) (end 122.1232 91.0002) (width 0.2) (layer "F.Cu") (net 8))
 (segment (start 122.9868 91.051) (end 123.244874 91.051) (width 0.2) (layer "F.Cu") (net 8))
 (segment (start 120.665199 91.567) (end 121.181199 91.051) (width 0.2) (layer "F.Cu") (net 8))
 (segment (start 120.665199 91.9734) (end 120.665199 91.567) (width 0.1524) (layer "F.Cu") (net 8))
 (segment (start 123.9423 87.9632) (end 123.3043 87.3252) (width 0.2) (layer "F.Cu") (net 8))
 (segment (start 123.9423 90.353574) (end 123.9423 87.9632) (width 0.2) (layer "F.Cu") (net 8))
 (segment (start 123.9892 87.3252) (end 124.8156 88.1516) (width 0.2) (layer "F.Cu") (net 8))
 (segment (start 123.244874 91.051) (end 123.9423 90.353574) (width 0.2) (layer "F.Cu") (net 8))
 (segment (start 122.1232 91.0002) (end 122.936 91.0002) (width 0.2) (layer "F.Cu") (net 8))
 (segment (start 122.936 91.0002) (end 122.9868 91.051) (width 0.1524) (layer "F.Cu") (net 8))
 (segment (start 123.3043 87.3252) (end 123.9892 87.3252) (width 0.2) (layer "F.Cu") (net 8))
 (segment (start 119.0244 92.3417) (end 119.0244 90.8431) (width 0.2) (layer "F.Cu") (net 3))
 (segment (start 120.4722 93.5736) (end 120.3198 93.5736) (width 0.1524) (layer "F.Cu") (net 3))
 (segment (start 120.3198 93.5736) (end 119.0244 92.2782) (width 0.2) (layer "F.Cu") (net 3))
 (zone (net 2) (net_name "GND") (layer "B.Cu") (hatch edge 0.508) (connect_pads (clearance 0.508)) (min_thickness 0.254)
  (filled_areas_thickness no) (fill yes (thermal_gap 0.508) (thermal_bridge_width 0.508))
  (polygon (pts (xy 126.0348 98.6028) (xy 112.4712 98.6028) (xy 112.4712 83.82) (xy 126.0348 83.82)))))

